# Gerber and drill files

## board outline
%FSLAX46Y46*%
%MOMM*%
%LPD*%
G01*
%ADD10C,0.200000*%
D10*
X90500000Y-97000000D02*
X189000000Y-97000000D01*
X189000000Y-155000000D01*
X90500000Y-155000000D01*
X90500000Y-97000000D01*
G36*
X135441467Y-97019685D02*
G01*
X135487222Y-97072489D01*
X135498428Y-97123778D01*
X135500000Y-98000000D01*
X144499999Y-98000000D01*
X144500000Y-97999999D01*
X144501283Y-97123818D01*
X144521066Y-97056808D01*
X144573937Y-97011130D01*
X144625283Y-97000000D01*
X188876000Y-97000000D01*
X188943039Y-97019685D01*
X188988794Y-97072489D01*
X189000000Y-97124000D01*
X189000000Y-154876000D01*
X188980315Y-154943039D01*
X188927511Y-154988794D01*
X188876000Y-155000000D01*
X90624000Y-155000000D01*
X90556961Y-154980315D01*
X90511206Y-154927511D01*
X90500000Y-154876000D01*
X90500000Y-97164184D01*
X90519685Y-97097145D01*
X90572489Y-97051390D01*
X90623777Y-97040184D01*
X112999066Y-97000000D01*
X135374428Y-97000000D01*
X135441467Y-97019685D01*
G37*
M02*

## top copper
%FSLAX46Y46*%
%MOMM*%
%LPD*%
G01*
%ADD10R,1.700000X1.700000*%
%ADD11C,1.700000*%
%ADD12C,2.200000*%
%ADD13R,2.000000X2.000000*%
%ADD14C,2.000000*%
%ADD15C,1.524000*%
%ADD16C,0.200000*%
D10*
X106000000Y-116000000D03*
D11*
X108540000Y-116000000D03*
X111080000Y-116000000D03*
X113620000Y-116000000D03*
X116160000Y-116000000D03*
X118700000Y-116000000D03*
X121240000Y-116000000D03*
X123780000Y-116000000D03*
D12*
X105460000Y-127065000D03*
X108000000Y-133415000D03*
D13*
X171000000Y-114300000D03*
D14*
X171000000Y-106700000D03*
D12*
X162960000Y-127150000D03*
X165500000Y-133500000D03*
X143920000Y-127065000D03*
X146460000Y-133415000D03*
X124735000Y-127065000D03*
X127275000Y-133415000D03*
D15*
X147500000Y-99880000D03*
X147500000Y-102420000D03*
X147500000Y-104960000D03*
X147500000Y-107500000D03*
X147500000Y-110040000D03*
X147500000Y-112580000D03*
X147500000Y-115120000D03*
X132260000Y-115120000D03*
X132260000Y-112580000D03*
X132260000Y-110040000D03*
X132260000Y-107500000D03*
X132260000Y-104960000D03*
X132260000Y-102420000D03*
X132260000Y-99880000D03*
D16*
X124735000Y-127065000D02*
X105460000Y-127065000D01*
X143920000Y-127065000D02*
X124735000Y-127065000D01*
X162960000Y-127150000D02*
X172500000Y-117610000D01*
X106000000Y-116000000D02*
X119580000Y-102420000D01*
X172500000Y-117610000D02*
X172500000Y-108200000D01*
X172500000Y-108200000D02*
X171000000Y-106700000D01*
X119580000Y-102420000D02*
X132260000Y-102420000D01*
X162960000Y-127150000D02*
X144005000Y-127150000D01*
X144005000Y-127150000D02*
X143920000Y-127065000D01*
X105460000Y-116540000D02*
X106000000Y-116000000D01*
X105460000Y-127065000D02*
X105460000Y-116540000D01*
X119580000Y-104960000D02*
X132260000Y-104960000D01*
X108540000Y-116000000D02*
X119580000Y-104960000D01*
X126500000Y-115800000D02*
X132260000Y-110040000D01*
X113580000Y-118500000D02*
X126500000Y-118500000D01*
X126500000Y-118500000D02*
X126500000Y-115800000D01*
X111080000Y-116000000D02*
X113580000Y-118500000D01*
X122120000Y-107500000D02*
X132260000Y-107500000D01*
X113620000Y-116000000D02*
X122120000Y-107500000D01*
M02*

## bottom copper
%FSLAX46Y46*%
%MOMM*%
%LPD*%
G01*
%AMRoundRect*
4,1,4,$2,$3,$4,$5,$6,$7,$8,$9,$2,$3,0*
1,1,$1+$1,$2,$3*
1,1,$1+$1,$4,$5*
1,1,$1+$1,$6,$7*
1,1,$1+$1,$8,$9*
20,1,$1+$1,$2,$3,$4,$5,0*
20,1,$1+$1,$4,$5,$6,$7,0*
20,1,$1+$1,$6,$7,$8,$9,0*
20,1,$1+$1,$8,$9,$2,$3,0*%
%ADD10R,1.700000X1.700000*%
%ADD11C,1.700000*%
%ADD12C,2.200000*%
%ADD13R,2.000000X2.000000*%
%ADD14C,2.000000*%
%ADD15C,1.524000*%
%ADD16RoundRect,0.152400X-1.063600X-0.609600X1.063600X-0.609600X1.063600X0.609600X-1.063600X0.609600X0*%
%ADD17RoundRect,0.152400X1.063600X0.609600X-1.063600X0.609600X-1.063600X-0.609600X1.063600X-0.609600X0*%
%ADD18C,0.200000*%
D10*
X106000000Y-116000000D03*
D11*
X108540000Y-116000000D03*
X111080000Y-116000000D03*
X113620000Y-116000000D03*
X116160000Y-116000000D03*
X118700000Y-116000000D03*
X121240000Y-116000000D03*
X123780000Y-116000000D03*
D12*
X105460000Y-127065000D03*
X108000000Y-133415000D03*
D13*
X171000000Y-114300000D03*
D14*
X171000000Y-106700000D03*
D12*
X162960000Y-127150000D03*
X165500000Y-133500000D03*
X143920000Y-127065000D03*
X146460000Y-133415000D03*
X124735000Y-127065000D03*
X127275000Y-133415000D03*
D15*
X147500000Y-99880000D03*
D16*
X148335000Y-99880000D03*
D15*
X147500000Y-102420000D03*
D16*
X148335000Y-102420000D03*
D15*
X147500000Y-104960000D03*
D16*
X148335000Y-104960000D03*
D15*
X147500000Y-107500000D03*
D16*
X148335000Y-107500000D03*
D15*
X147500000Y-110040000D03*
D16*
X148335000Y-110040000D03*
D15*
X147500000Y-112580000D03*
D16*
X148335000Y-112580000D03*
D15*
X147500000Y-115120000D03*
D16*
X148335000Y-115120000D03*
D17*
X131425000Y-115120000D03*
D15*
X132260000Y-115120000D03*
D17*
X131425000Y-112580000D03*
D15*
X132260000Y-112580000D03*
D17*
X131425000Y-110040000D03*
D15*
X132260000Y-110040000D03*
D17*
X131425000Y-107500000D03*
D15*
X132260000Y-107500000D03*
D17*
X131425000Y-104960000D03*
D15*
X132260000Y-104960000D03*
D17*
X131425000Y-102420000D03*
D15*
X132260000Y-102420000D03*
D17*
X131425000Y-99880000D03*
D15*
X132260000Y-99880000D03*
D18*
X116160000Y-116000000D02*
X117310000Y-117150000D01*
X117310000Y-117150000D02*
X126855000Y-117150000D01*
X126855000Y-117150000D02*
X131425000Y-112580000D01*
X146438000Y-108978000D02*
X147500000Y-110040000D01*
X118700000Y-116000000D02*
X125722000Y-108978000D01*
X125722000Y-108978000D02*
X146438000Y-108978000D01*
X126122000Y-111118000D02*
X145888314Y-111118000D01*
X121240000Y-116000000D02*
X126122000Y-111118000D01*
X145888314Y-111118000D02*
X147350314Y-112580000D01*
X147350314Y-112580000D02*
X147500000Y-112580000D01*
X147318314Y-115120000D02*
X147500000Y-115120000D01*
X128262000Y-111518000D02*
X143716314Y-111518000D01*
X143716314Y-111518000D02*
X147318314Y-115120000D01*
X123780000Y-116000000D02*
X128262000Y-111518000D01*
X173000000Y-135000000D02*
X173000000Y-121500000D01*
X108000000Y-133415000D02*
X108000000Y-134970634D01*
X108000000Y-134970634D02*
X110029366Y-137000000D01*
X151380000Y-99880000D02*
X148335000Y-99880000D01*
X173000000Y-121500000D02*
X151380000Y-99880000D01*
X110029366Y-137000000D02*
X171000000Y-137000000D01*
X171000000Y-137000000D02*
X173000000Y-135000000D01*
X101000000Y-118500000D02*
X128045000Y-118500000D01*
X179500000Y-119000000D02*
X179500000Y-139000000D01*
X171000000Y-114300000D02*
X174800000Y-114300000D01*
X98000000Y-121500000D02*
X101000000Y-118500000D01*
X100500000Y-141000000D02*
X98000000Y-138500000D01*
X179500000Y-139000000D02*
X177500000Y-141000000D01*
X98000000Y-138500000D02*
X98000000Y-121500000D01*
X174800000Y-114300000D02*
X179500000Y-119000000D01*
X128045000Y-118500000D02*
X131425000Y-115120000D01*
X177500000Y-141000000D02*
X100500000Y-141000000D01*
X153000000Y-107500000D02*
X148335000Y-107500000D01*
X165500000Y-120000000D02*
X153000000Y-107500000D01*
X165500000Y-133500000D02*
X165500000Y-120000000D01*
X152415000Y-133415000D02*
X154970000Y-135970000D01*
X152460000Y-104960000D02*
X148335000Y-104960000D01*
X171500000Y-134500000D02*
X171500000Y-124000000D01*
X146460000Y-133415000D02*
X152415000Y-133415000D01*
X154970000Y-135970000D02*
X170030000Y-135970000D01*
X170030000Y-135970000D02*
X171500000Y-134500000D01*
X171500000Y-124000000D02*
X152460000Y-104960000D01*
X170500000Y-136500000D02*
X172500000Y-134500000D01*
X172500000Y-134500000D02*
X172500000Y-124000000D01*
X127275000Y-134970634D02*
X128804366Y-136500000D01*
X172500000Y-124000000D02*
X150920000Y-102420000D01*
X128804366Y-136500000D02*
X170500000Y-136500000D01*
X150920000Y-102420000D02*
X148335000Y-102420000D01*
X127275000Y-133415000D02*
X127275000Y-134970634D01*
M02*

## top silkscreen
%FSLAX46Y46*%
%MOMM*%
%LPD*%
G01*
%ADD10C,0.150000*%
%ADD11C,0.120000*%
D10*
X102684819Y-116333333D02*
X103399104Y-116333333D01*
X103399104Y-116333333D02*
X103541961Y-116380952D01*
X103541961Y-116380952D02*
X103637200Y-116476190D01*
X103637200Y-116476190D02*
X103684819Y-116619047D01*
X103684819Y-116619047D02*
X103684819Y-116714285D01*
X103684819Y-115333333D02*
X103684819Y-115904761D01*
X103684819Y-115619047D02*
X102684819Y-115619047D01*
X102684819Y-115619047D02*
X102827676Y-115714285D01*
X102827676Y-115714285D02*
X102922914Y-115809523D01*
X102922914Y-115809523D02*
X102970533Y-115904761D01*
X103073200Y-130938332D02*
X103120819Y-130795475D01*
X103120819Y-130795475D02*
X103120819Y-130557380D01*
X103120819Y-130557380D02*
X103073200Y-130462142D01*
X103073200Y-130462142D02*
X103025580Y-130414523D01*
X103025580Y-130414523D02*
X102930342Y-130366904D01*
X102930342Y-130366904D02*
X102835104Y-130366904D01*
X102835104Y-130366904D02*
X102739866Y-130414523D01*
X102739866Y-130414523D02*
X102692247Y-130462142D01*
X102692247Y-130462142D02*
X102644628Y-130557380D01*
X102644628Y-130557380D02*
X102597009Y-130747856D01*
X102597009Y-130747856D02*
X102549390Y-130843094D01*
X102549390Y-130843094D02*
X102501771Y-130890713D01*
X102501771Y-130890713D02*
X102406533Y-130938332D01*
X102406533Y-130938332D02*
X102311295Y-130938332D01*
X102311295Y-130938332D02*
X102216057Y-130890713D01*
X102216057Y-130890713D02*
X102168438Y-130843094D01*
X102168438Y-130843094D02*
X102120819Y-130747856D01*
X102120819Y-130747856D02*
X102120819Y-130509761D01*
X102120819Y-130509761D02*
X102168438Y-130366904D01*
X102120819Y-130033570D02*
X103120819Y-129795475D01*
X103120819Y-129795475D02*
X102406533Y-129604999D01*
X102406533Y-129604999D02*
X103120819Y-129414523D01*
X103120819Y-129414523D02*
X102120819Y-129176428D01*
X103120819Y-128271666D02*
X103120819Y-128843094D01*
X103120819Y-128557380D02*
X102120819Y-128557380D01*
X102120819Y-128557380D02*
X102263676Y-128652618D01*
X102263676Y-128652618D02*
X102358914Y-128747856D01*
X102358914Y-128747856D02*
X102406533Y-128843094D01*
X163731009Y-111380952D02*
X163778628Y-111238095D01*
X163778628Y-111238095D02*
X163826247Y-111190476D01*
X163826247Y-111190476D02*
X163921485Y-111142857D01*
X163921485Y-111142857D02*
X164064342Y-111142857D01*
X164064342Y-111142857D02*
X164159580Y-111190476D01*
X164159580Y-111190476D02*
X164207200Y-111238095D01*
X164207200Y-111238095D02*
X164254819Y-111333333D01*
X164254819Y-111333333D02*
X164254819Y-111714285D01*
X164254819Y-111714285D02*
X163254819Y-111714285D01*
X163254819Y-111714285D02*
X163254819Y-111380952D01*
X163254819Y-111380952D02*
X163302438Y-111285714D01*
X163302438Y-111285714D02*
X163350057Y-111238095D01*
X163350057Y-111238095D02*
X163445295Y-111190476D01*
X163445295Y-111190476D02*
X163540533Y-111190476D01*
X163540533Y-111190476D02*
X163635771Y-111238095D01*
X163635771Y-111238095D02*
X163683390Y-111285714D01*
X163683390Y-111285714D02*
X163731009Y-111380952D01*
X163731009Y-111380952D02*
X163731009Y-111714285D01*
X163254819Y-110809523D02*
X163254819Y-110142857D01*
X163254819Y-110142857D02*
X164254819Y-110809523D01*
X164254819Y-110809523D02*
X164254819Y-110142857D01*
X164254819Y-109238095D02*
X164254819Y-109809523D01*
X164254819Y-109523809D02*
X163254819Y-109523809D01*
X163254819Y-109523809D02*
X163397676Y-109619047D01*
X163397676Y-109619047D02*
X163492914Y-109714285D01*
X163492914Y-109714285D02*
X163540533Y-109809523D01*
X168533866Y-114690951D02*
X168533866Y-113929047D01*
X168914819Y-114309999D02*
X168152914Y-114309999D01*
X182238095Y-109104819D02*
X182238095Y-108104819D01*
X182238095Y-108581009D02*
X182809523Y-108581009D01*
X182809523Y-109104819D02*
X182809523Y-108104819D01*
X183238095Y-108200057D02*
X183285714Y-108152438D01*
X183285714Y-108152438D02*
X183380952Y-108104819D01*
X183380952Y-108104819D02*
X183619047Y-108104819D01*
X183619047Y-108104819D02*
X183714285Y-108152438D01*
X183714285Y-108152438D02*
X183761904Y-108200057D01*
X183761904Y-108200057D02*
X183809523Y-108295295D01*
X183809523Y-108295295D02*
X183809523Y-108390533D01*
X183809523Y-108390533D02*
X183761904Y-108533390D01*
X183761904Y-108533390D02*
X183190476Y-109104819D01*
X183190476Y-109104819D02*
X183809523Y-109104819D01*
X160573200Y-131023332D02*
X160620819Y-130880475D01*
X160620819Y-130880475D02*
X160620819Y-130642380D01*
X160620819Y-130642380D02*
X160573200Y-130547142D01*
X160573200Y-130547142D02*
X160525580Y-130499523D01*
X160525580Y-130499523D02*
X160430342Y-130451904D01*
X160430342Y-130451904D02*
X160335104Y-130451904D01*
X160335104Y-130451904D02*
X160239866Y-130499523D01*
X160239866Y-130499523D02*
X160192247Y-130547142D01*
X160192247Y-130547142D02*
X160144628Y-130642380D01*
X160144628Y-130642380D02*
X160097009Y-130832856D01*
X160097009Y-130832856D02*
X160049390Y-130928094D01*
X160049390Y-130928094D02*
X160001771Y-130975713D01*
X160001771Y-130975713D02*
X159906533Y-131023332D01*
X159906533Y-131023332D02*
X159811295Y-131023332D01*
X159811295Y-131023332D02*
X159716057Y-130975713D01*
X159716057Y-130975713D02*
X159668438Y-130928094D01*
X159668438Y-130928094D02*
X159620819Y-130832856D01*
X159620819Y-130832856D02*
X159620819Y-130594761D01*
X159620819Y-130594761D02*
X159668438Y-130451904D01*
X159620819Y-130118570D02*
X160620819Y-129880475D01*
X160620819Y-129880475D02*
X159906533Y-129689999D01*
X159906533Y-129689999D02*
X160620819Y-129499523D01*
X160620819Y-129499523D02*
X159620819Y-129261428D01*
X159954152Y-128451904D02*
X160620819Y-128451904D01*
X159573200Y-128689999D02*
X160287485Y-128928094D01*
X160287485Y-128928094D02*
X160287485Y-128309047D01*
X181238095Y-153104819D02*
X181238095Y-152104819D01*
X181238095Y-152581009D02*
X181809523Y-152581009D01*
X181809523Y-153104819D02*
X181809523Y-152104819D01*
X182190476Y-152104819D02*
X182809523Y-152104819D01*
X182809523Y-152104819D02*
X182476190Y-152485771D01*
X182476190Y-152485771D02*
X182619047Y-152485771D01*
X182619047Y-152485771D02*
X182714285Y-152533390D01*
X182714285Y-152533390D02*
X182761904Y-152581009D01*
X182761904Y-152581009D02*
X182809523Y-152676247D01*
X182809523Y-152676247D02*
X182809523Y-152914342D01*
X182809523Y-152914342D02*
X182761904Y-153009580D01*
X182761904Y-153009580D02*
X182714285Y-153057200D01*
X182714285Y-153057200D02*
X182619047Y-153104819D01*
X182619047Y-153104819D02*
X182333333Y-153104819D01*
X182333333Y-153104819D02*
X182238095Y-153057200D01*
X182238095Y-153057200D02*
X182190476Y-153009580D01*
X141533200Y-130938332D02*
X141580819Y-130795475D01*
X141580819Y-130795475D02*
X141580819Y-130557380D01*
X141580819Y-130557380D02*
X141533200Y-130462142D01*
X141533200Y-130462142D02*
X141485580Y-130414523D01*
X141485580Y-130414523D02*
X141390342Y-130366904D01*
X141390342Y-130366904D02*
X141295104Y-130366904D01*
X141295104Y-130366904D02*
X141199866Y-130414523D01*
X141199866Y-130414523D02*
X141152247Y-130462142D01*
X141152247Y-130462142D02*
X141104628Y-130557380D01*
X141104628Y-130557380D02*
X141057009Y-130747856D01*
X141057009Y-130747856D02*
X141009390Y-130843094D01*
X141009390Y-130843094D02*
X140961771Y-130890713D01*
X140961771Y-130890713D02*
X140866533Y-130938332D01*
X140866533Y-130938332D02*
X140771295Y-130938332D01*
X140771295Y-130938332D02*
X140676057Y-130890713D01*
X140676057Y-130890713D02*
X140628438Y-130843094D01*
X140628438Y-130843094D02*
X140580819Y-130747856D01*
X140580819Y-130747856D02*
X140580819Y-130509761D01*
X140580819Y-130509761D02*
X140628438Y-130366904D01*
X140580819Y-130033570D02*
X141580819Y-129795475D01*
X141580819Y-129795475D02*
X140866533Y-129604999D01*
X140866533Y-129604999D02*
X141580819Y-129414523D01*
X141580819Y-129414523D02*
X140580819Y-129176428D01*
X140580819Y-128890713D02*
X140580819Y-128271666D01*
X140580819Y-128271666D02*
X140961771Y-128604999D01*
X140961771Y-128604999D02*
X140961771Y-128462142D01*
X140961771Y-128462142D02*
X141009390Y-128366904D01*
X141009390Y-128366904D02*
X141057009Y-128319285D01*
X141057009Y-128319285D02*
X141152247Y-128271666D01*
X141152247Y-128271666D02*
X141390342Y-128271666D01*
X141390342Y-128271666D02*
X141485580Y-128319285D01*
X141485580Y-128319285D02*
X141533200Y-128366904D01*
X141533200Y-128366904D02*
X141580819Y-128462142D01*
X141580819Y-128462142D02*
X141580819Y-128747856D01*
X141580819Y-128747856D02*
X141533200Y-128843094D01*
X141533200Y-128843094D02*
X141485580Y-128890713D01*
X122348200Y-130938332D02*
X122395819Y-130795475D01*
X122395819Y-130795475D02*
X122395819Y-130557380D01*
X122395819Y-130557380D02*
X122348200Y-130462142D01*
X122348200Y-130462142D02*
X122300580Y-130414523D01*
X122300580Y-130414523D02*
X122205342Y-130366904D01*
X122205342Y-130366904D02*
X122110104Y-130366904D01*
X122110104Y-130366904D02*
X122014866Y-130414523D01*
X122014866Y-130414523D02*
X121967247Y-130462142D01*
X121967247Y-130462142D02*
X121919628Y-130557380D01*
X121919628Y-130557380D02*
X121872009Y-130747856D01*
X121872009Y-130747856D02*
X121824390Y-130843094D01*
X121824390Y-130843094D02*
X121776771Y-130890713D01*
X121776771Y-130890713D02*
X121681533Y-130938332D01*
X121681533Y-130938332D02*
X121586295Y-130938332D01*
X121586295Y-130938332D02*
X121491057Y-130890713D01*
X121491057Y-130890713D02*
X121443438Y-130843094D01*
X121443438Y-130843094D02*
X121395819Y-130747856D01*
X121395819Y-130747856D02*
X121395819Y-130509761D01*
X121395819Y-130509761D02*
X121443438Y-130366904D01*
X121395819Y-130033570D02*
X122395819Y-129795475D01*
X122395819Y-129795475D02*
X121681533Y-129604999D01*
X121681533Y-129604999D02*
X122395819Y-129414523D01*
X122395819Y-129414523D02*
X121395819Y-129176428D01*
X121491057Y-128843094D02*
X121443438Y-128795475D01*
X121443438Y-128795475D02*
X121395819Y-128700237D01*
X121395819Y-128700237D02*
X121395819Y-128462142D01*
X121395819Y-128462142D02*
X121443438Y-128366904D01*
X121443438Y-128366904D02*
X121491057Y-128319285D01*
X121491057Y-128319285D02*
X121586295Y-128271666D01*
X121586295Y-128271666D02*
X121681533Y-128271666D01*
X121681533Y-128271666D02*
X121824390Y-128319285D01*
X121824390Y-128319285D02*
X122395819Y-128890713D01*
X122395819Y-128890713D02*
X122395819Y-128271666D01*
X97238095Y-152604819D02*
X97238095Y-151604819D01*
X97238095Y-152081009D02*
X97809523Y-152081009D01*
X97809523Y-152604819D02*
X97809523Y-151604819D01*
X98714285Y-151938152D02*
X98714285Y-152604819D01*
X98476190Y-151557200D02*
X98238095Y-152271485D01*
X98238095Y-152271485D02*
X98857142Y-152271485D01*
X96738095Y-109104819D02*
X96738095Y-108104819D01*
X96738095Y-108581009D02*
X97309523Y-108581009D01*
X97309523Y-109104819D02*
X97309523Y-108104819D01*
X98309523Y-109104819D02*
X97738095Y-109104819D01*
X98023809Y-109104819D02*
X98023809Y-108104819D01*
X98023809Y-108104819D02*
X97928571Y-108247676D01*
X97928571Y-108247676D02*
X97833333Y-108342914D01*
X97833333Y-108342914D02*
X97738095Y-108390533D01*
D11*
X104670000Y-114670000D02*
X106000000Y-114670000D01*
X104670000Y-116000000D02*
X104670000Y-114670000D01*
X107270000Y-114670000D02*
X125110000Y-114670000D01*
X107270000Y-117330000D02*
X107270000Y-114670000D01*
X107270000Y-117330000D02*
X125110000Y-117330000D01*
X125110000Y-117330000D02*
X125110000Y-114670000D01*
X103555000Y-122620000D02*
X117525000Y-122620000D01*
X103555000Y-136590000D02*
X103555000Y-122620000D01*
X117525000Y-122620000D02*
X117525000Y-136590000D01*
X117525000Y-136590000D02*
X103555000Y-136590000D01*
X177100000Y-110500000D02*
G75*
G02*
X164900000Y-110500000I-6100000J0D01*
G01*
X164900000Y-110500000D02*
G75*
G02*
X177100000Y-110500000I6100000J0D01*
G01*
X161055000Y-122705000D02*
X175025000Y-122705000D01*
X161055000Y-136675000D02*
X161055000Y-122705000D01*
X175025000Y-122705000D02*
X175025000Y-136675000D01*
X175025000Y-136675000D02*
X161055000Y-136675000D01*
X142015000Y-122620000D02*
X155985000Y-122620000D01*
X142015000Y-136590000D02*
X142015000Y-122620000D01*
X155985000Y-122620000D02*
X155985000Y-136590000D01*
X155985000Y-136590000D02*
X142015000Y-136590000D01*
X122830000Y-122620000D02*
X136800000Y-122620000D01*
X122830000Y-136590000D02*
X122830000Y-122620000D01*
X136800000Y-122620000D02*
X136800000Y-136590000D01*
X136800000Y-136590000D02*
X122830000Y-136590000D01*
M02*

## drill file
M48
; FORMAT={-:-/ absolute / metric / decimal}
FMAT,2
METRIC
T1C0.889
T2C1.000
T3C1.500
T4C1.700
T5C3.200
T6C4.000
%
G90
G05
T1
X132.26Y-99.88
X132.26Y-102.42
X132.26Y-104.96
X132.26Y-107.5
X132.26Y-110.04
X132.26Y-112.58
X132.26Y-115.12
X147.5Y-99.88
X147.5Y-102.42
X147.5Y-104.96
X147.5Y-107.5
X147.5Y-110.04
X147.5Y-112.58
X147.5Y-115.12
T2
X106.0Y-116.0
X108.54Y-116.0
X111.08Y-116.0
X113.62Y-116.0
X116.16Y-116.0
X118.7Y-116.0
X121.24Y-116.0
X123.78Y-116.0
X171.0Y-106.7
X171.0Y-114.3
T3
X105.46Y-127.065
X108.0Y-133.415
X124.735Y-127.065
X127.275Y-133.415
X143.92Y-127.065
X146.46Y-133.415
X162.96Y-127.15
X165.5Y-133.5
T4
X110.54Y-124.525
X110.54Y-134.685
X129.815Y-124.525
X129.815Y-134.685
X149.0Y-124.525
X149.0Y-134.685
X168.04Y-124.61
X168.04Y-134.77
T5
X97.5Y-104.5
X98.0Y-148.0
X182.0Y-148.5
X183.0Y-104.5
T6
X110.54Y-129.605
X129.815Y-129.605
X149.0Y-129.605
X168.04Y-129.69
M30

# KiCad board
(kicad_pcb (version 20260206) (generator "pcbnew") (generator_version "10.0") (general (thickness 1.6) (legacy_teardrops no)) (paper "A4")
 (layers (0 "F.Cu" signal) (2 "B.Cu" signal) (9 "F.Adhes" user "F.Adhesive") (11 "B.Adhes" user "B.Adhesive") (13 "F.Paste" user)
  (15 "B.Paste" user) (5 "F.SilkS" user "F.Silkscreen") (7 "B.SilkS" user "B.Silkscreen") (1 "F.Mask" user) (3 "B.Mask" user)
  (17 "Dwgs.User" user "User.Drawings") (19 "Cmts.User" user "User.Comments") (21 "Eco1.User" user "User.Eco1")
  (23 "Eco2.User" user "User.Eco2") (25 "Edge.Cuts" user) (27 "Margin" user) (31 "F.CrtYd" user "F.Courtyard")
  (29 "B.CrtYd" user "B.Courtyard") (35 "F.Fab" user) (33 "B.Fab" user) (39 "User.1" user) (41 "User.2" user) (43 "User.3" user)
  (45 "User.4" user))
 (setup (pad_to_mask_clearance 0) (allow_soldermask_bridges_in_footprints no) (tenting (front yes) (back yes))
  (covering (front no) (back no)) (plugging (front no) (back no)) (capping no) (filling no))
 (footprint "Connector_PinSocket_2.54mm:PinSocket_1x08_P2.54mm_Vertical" (layer "F.Cu") (at 106 116 90)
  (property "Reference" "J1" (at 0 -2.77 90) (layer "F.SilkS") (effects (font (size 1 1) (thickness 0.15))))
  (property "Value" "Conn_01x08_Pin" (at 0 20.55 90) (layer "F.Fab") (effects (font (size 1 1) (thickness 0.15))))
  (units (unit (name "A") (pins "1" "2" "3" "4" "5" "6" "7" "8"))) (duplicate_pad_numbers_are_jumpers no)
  (fp_line (start 1.33 -1.33) (end 1.33 0) (stroke (width 0.12) (type solid)) (layer "F.SilkS"))
  (fp_line (start 0 -1.33) (end 1.33 -1.33) (stroke (width 0.12) (type solid)) (layer "F.SilkS"))
  (fp_line (start 1.33 1.27) (end 1.33 19.11) (stroke (width 0.12) (type solid)) (layer "F.SilkS"))
  (fp_line (start -1.33 1.27) (end 1.33 1.27) (stroke (width 0.12) (type solid)) (layer "F.SilkS"))
  (fp_line (start -1.33 1.27) (end -1.33 19.11) (stroke (width 0.12) (type solid)) (layer "F.SilkS"))
  (fp_line (start -1.33 19.11) (end 1.33 19.11) (stroke (width 0.12) (type solid)) (layer "F.SilkS"))
  (pad "1" thru_hole rect (at 0 0 90) (size 1.7 1.7) (drill 1) (layers "*.Cu" "*.Mask") (remove_unused_layers no) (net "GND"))
  (pad "2" thru_hole circle (at 0 2.54 90) (size 1.7 1.7) (drill 1) (layers "*.Cu" "*.Mask") (remove_unused_layers no) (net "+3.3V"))
  (pad "3" thru_hole circle (at 0 5.08 90) (size 1.7 1.7) (drill 1) (layers "*.Cu" "*.Mask") (remove_unused_layers no) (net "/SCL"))
  (pad "4" thru_hole circle (at 0 7.62 90) (size 1.7 1.7) (drill 1) (layers "*.Cu" "*.Mask") (remove_unused_layers no) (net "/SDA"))
  (pad "5" thru_hole circle (at 0 10.16 90) (size 1.7 1.7) (drill 1) (layers "*.Cu" "*.Mask") (remove_unused_layers no) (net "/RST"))
  (pad "6" thru_hole circle (at 0 12.7 90) (size 1.7 1.7) (drill 1) (layers "*.Cu" "*.Mask") (remove_unused_layers no) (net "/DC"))
  (pad "7" thru_hole circle (at 0 15.24 90) (size 1.7 1.7) (drill 1) (layers "*.Cu" "*.Mask") (remove_unused_layers no) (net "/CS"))
  (pad "8" thru_hole circle (at 0 17.78 90) (size 1.7 1.7) (drill 1) (layers "*.Cu" "*.Mask") (remove_unused_layers no) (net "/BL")))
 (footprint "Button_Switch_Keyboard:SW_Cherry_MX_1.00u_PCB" (layer "F.Cu") (at 105.46 127.065 90)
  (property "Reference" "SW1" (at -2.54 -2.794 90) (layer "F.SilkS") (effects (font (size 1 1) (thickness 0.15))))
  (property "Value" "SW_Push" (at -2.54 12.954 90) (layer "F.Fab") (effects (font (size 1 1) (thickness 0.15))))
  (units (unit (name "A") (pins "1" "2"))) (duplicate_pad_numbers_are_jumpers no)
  (fp_line (start 4.445 -1.905) (end 4.445 12.065) (stroke (width 0.12) (type solid)) (layer "F.SilkS"))
  (fp_line (start -9.525 -1.905) (end 4.445 -1.905) (stroke (width 0.12) (type solid)) (layer "F.SilkS"))
  (fp_line (start 4.445 12.065) (end -9.525 12.065) (stroke (width 0.12) (type solid)) (layer "F.SilkS"))
  (fp_line (start -9.525 12.065) (end -9.525 -1.905) (stroke (width 0.12) (type solid)) (layer "F.SilkS"))
  (pad "" np_thru_hole circle (at -7.62 5.08 90) (size 1.7 1.7) (drill 1.7) (layers "*.Cu" "*.Mask"))
  (pad "" np_thru_hole circle (at -2.54 5.08 90) (size 4 4) (drill 4) (layers "*.Cu" "*.Mask"))
  (pad "" np_thru_hole circle (at 2.54 5.08 90) (size 1.7 1.7) (drill 1.7) (layers "*.Cu" "*.Mask"))
  (pad "1" thru_hole circle (at 0 0 90) (size 2.2 2.2) (drill 1.5) (layers "*.Cu" "*.Mask") (remove_unused_layers no) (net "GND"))
  (pad "2" thru_hole circle (at -6.35 2.54 90) (size 2.2 2.2) (drill 1.5) (layers "*.Cu" "*.Mask") (remove_unused_layers no)
   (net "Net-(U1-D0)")))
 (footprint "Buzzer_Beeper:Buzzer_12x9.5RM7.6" (layer "F.Cu") (at 171 114.3 90)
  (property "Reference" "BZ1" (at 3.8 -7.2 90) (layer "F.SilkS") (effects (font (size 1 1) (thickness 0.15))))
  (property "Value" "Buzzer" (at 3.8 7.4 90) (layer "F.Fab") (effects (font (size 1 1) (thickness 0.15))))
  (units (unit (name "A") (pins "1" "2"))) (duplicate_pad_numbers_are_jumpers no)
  (fp_circle (center 3.8 0) (end 9.9 0) (stroke (width 0.12) (type solid)) (fill no) (layer "F.SilkS"))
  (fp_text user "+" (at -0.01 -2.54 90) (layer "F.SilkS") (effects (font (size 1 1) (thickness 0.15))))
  (pad "1" thru_hole rect (at 0 0 90) (size 2 2) (drill 1) (layers "*.Cu" "*.Mask") (remove_unused_layers no) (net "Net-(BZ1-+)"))
  (pad "2" thru_hole circle (at 7.6 0 90) (size 2 2) (drill 1) (layers "*.Cu" "*.Mask") (remove_unused_layers no) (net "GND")))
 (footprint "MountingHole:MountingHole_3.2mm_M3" (layer "F.Cu") (at 183 104.5 180)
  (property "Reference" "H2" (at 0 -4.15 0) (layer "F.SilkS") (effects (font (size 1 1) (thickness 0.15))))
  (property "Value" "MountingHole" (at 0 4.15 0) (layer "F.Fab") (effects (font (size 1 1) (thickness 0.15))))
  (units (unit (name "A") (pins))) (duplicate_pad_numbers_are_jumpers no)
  (pad "" np_thru_hole circle (at 0 0 180) (size 3.2 3.2) (drill 3.2) (layers "*.Cu" "*.Mask")))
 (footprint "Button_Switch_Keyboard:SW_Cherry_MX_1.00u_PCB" (layer "F.Cu") (at 162.96 127.15 90)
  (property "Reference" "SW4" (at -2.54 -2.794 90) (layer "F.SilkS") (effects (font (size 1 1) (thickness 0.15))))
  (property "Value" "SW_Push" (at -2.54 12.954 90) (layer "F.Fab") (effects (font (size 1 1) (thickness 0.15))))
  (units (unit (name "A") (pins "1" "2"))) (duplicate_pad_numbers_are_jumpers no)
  (fp_line (start 4.445 -1.905) (end 4.445 12.065) (stroke (width 0.12) (type solid)) (layer "F.SilkS"))
  (fp_line (start -9.525 -1.905) (end 4.445 -1.905) (stroke (width 0.12) (type solid)) (layer "F.SilkS"))
  (fp_line (start 4.445 12.065) (end -9.525 12.065) (stroke (width 0.12) (type solid)) (layer "F.SilkS"))
  (fp_line (start -9.525 12.065) (end -9.525 -1.905) (stroke (width 0.12) (type solid)) (layer "F.SilkS"))
  (pad "" np_thru_hole circle (at -7.62 5.08 90) (size 1.7 1.7) (drill 1.7) (layers "*.Cu" "*.Mask"))
  (pad "" np_thru_hole circle (at -2.54 5.08 90) (size 4 4) (drill 4) (layers "*.Cu" "*.Mask"))
  (pad "" np_thru_hole circle (at 2.54 5.08 90) (size 1.7 1.7) (drill 1.7) (layers "*.Cu" "*.Mask"))
  (pad "1" thru_hole circle (at 0 0 90) (size 2.2 2.2) (drill 1.5) (layers "*.Cu" "*.Mask") (remove_unused_layers no) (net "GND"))
  (pad "2" thru_hole circle (at -6.35 2.54 90) (size 2.2 2.2) (drill 1.5) (layers "*.Cu" "*.Mask") (remove_unused_layers no)
   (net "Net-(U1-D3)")))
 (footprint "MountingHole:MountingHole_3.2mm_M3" (layer "F.Cu") (at 182 148.5 180)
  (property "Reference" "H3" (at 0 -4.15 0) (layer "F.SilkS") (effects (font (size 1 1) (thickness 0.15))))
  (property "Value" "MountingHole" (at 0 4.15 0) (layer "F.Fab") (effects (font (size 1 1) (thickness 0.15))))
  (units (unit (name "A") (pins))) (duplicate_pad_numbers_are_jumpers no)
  (pad "" np_thru_hole circle (at 0 0 180) (size 3.2 3.2) (drill 3.2) (layers "*.Cu" "*.Mask")))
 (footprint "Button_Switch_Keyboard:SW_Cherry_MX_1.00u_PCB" (layer "F.Cu") (at 143.92 127.065 90)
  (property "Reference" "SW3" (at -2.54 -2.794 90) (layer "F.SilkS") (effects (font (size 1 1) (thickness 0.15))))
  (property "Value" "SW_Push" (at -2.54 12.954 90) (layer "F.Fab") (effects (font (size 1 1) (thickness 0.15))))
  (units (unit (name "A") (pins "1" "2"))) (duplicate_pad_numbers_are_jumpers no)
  (fp_line (start 4.445 -1.905) (end 4.445 12.065) (stroke (width 0.12) (type solid)) (layer "F.SilkS"))
  (fp_line (start -9.525 -1.905) (end 4.445 -1.905) (stroke (width 0.12) (type solid)) (layer "F.SilkS"))
  (fp_line (start 4.445 12.065) (end -9.525 12.065) (stroke (width 0.12) (type solid)) (layer "F.SilkS"))
  (fp_line (start -9.525 12.065) (end -9.525 -1.905) (stroke (width 0.12) (type solid)) (layer "F.SilkS"))
  (pad "" np_thru_hole circle (at -7.62 5.08 90) (size 1.7 1.7) (drill 1.7) (layers "*.Cu" "*.Mask"))
  (pad "" np_thru_hole circle (at -2.54 5.08 90) (size 4 4) (drill 4) (layers "*.Cu" "*.Mask"))
  (pad "" np_thru_hole circle (at 2.54 5.08 90) (size 1.7 1.7) (drill 1.7) (layers "*.Cu" "*.Mask"))
  (pad "1" thru_hole circle (at 0 0 90) (size 2.2 2.2) (drill 1.5) (layers "*.Cu" "*.Mask") (remove_unused_layers no) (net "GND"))
  (pad "2" thru_hole circle (at -6.35 2.54 90) (size 2.2 2.2) (drill 1.5) (layers "*.Cu" "*.Mask") (remove_unused_layers no)
   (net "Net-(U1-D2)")))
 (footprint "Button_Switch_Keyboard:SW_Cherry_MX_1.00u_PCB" (layer "F.Cu") (at 124.735 127.065 90)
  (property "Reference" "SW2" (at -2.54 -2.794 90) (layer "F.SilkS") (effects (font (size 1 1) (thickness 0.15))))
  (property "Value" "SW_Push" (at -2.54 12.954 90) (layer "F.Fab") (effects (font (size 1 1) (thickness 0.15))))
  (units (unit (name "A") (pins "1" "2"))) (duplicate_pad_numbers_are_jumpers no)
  (fp_line (start 4.445 -1.905) (end 4.445 12.065) (stroke (width 0.12) (type solid)) (layer "F.SilkS"))
  (fp_line (start -9.525 -1.905) (end 4.445 -1.905) (stroke (width 0.12) (type solid)) (layer "F.SilkS"))
  (fp_line (start 4.445 12.065) (end -9.525 12.065) (stroke (width 0.12) (type solid)) (layer "F.SilkS"))
  (fp_line (start -9.525 12.065) (end -9.525 -1.905) (stroke (width 0.12) (type solid)) (layer "F.SilkS"))
  (pad "" np_thru_hole circle (at -7.62 5.08 90) (size 1.7 1.7) (drill 1.7) (layers "*.Cu" "*.Mask"))
  (pad "" np_thru_hole circle (at -2.54 5.08 90) (size 4 4) (drill 4) (layers "*.Cu" "*.Mask"))
  (pad "" np_thru_hole circle (at 2.54 5.08 90) (size 1.7 1.7) (drill 1.7) (layers "*.Cu" "*.Mask"))
  (pad "1" thru_hole circle (at 0 0 90) (size 2.2 2.2) (drill 1.5) (layers "*.Cu" "*.Mask") (remove_unused_layers no) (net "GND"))
  (pad "2" thru_hole circle (at -6.35 2.54 90) (size 2.2 2.2) (drill 1.5) (layers "*.Cu" "*.Mask") (remove_unused_layers no)
   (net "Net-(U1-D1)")))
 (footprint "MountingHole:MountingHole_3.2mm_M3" (layer "F.Cu") (at 98 148 180)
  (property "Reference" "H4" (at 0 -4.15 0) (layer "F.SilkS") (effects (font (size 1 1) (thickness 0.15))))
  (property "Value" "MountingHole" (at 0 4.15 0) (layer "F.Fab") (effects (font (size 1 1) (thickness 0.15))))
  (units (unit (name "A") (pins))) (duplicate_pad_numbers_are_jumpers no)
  (pad "" np_thru_hole circle (at 0 0 180) (size 3.2 3.2) (drill 3.2) (layers "*.Cu" "*.Mask")))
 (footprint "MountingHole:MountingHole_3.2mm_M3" (layer "F.Cu") (at 97.5 104.5 180)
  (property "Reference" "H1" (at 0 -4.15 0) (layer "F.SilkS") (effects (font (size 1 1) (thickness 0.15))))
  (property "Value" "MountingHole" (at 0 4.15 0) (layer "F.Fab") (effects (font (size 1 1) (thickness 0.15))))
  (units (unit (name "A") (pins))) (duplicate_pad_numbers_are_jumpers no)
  (pad "" np_thru_hole circle (at 0 0 180) (size 3.2 3.2) (drill 3.2) (layers "*.Cu" "*.Mask")))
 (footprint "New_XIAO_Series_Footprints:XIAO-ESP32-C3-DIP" (layer "B.Cu") (at 139.88 107.5 90)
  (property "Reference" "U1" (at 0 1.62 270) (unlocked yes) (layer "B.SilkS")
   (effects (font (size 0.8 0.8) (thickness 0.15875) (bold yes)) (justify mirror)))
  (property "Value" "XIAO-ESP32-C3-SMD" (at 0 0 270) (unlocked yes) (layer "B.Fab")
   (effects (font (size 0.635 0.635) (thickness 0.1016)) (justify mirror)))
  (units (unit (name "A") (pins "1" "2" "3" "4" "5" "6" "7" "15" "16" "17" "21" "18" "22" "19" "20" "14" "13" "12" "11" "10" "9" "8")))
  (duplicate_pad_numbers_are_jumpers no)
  (pad "1" thru_hole circle (at 7.62 7.62) (size 1.524 1.524) (drill 0.889) (layers "*.Cu" "*.Mask") (remove_unused_layers no)
   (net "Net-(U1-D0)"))
  (pad "1" smd roundrect (at 7.62 8.455) (size 2.432 1.524) (layers "B.Cu" "B.Mask") (roundrect_rratio 0.1) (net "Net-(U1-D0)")
   (thermal_bridge_angle 45))
  (pad "2" thru_hole circle (at 5.08 7.62) (size 1.524 1.524) (drill 0.889) (layers "*.Cu" "*.Mask") (remove_unused_layers no)
   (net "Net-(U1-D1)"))
  (pad "2" smd roundrect (at 5.08 8.455) (size 2.432 1.524) (layers "B.Cu" "B.Mask") (roundrect_rratio 0.1) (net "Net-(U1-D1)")
   (thermal_bridge_angle 45))
  (pad "3" thru_hole circle (at 2.54 7.62) (size 1.524 1.524) (drill 0.889) (layers "*.Cu" "*.Mask") (remove_unused_layers no)
   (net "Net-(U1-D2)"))
  (pad "3" smd roundrect (at 2.54 8.455) (size 2.432 1.524) (layers "B.Cu" "B.Mask") (roundrect_rratio 0.1) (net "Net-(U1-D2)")
   (thermal_bridge_angle 45))
  (pad "4" thru_hole circle (at 0 7.62) (size 1.524 1.524) (drill 0.889) (layers "*.Cu" "*.Mask") (remove_unused_layers no)
   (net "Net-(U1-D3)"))
  (pad "4" smd roundrect (at 0 8.455) (size 2.432 1.524) (layers "B.Cu" "B.Mask") (roundrect_rratio 0.1) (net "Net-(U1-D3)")
   (thermal_bridge_angle 45))
  (pad "5" thru_hole circle (at -2.54 7.62) (size 1.524 1.524) (drill 0.889) (layers "*.Cu" "*.Mask") (remove_unused_layers no) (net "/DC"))
  (pad "5" smd roundrect (at -2.54 8.455) (size 2.432 1.524) (layers "B.Cu" "B.Mask") (roundrect_rratio 0.1) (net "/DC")
   (thermal_bridge_angle 45))
  (pad "6" thru_hole circle (at -5.08 7.62) (size 1.524 1.524) (drill 0.889) (layers "*.Cu" "*.Mask") (remove_unused_layers no) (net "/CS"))
  (pad "6" smd roundrect (at -5.08 8.455) (size 2.432 1.524) (layers "B.Cu" "B.Mask") (roundrect_rratio 0.1) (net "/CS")
   (thermal_bridge_angle 45))
  (pad "7" thru_hole circle (at -7.62 7.62) (size 1.524 1.524) (drill 0.889) (layers "*.Cu" "*.Mask") (remove_unused_layers no) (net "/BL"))
  (pad "7" smd roundrect (at -7.62 8.455) (size 2.432 1.524) (layers "B.Cu" "B.Mask") (roundrect_rratio 0.1) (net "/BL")
   (thermal_bridge_angle 45))
  (pad "8" smd roundrect (at -7.62 -8.455 180) (size 2.432 1.524) (layers "B.Cu" "B.Mask") (roundrect_rratio 0.1) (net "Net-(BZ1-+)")
   (thermal_bridge_angle 45))
  (pad "8" thru_hole circle (at -7.62 -7.62 180) (size 1.524 1.524) (drill 0.889) (layers "*.Cu" "*.Mask") (remove_unused_layers no)
   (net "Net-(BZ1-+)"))
  (pad "9" smd roundrect (at -5.08 -8.455 180) (size 2.432 1.524) (layers "B.Cu" "B.Mask") (roundrect_rratio 0.1) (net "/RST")
   (thermal_bridge_angle 45))
  (pad "9" thru_hole circle (at -5.08 -7.62 180) (size 1.524 1.524) (drill 0.889) (layers "*.Cu" "*.Mask") (remove_unused_layers no)
   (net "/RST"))
  (pad "10" smd roundrect (at -2.54 -8.455 180) (size 2.432 1.524) (layers "B.Cu" "B.Mask") (roundrect_rratio 0.1) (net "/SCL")
   (thermal_bridge_angle 45))
  (pad "10" thru_hole circle (at -2.54 -7.62 180) (size 1.524 1.524) (drill 0.889) (layers "*.Cu" "*.Mask") (remove_unused_layers no)
   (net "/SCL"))
  (pad "11" smd roundrect (at 0 -8.455 180) (size 2.432 1.524) (layers "B.Cu" "B.Mask") (roundrect_rratio 0.1) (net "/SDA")
   (thermal_bridge_angle 45))
  (pad "11" thru_hole circle (at 0 -7.62 180) (size 1.524 1.524) (drill 0.889) (layers "*.Cu" "*.Mask") (remove_unused_layers no)
   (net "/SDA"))
  (pad "12" smd roundrect (at 2.54 -8.455 180) (size 2.432 1.524) (layers "B.Cu" "B.Mask") (roundrect_rratio 0.1) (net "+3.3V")
   (thermal_bridge_angle 45))
  (pad "12" thru_hole circle (at 2.54 -7.62 180) (size 1.524 1.524) (drill 0.889) (layers "*.Cu" "*.Mask") (remove_unused_layers no)
   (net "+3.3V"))
  (pad "13" smd roundrect (at 5.08 -8.455 180) (size 2.432 1.524) (layers "B.Cu" "B.Mask") (roundrect_rratio 0.1) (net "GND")
   (thermal_bridge_angle 45))
  (pad "13" thru_hole circle (at 5.08 -7.62 180) (size 1.524 1.524) (drill 0.889) (layers "*.Cu" "*.Mask") (remove_unused_layers no)
   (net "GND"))
  (pad "14" smd roundrect (at 7.62 -8.455 180) (size 2.432 1.524) (layers "B.Cu" "B.Mask") (roundrect_rratio 0.1)
   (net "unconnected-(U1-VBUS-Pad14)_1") (thermal_bridge_angle 45))
  (pad "14" thru_hole circle (at 7.62 -7.62 180) (size 1.524 1.524) (drill 0.889) (layers "*.Cu" "*.Mask") (remove_unused_layers no)
   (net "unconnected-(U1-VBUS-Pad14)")))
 (gr_rect (start 90.5 97) (end 189 155) (stroke (width 0.2) (type default)) (fill no) (layer "Edge.Cuts"))
 (segment (start 124.735 127.065) (end 105.46 127.065) (width 0.2) (layer "F.Cu") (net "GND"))
 (segment (start 143.92 127.065) (end 124.735 127.065) (width 0.2) (layer "F.Cu") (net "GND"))
 (segment (start 162.96 127.15) (end 172.5 117.61) (width 0.2) (layer "F.Cu") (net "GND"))
 (segment (start 106 116) (end 119.58 102.42) (width 0.2) (layer "F.Cu") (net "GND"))
 (segment (start 172.5 117.61) (end 172.5 108.2) (width 0.2) (layer "F.Cu") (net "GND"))
 (segment (start 172.5 108.2) (end 171 106.7) (width 0.2) (layer "F.Cu") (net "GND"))
 (segment (start 119.58 102.42) (end 132.26 102.42) (width 0.2) (layer "F.Cu") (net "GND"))
 (segment (start 162.96 127.15) (end 144.005 127.15) (width 0.2) (layer "F.Cu") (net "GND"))
 (segment (start 144.005 127.15) (end 143.92 127.065) (width 0.2) (layer "F.Cu") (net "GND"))
 (segment (start 105.46 116.54) (end 106 116) (width 0.2) (layer "F.Cu") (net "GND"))
 (segment (start 105.46 127.065) (end 105.46 116.54) (width 0.2) (layer "F.Cu") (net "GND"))
 (segment (start 119.58 104.96) (end 132.26 104.96) (width 0.2) (layer "F.Cu") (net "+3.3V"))
 (segment (start 108.54 116) (end 119.58 104.96) (width 0.2) (layer "F.Cu") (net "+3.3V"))
 (segment (start 126.5 115.8) (end 132.26 110.04) (width 0.2) (layer "F.Cu") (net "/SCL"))
 (segment (start 113.58 118.5) (end 126.5 118.5) (width 0.2) (layer "F.Cu") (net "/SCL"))
 (segment (start 126.5 118.5) (end 126.5 115.8) (width 0.2) (layer "F.Cu") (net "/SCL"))
 (segment (start 111.08 116) (end 113.58 118.5) (width 0.2) (layer "F.Cu") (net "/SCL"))
 (segment (start 122.12 107.5) (end 132.26 107.5) (width 0.2) (layer "F.Cu") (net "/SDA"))
 (segment (start 113.62 116) (end 122.12 107.5) (width 0.2) (layer "F.Cu") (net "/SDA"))
 (segment (start 116.16 116) (end 117.31 117.15) (width 0.2) (layer "B.Cu") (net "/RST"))
 (segment (start 117.31 117.15) (end 126.855 117.15) (width 0.2) (layer "B.Cu") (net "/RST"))
 (segment (start 126.855 117.15) (end 131.425 112.58) (width 0.2) (layer "B.Cu") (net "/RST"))
 (segment (start 146.438 108.978) (end 147.5 110.04) (width 0.2) (layer "B.Cu") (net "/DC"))
 (segment (start 118.7 116) (end 125.722 108.978) (width 0.2) (layer "B.Cu") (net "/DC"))
 (segment (start 125.722 108.978) (end 146.438 108.978) (width 0.2) (layer "B.Cu") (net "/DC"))
 (segment (start 126.122 111.118) (end 145.888314 111.118) (width 0.2) (layer "B.Cu") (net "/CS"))
 (segment (start 121.24 116) (end 126.122 111.118) (width 0.2) (layer "B.Cu") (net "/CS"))
 (segment (start 145.888314 111.118) (end 147.350314 112.58) (width 0.2) (layer "B.Cu") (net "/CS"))
 (segment (start 147.350314 112.58) (end 147.5 112.58) (width 0.2) (layer "B.Cu") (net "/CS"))
 (segment (start 147.318314 115.12) (end 147.5 115.12) (width 0.2) (layer "B.Cu") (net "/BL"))
 (segment (start 128.262 111.518) (end 143.716314 111.518) (width 0.2) (layer "B.Cu") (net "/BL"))
 (segment (start 143.716314 111.518) (end 147.318314 115.12) (width 0.2) (layer "B.Cu") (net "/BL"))
 (segment (start 123.78 116) (end 128.262 111.518) (width 0.2) (layer "B.Cu") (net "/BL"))
 (segment (start 173 135) (end 173 121.5) (width 0.2) (layer "B.Cu") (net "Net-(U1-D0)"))
 (segment (start 108 133.415) (end 108 134.970634) (width 0.2) (layer "B.Cu") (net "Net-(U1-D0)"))
 (segment (start 108 134.970634) (end 110.029366 137) (width 0.2) (layer "B.Cu") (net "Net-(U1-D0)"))
 (segment (start 151.38 99.88) (end 148.335 99.88) (width 0.2) (layer "B.Cu") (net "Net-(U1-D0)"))
 (segment (start 173 121.5) (end 151.38 99.88) (width 0.2) (layer "B.Cu") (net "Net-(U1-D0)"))
 (segment (start 110.029366 137) (end 171 137) (width 0.2) (layer "B.Cu") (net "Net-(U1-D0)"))
 (segment (start 171 137) (end 173 135) (width 0.2) (layer "B.Cu") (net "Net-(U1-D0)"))
 (segment (start 101 118.5) (end 128.045 118.5) (width 0.2) (layer "B.Cu") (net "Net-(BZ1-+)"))
 (segment (start 179.5 119) (end 179.5 139) (width 0.2) (layer "B.Cu") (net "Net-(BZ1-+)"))
 (segment (start 171 114.3) (end 174.8 114.3) (width 0.2) (layer "B.Cu") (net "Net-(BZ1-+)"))
 (segment (start 98 121.5) (end 101 118.5) (width 0.2) (layer "B.Cu") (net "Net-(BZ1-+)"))
 (segment (start 100.5 141) (end 98 138.5) (width 0.2) (layer "B.Cu") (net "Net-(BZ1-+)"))
 (segment (start 179.5 139) (end 177.5 141) (width 0.2) (layer "B.Cu") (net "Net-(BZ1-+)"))
 (segment (start 98 138.5) (end 98 121.5) (width 0.2) (layer "B.Cu") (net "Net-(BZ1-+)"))
 (segment (start 174.8 114.3) (end 179.5 119) (width 0.2) (layer "B.Cu") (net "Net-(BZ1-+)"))
 (segment (start 128.045 118.5) (end 131.425 115.12) (width 0.2) (layer "B.Cu") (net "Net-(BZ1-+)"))
 (segment (start 177.5 141) (end 100.5 141) (width 0.2) (layer "B.Cu") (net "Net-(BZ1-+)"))
 (segment (start 153 107.5) (end 148.335 107.5) (width 0.2) (layer "B.Cu") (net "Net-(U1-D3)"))
 (segment (start 165.5 120) (end 153 107.5) (width 0.2) (layer "B.Cu") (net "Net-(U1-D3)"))
 (segment (start 165.5 133.5) (end 165.5 120) (width 0.2) (layer "B.Cu") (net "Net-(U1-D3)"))
 (segment (start 152.415 133.415) (end 154.97 135.97) (width 0.2) (layer "B.Cu") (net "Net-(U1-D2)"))
 (segment (start 152.46 104.96) (end 148.335 104.96) (width 0.2) (layer "B.Cu") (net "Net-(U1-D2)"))
 (segment (start 171.5 134.5) (end 171.5 124) (width 0.2) (layer "B.Cu") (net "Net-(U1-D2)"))
 (segment (start 146.46 133.415) (end 152.415 133.415) (width 0.2) (layer "B.Cu") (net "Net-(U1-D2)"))
 (segment (start 154.97 135.97) (end 170.03 135.97) (width 0.2) (layer "B.Cu") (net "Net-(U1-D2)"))
 (segment (start 170.03 135.97) (end 171.5 134.5) (width 0.2) (layer "B.Cu") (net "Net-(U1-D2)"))
 (segment (start 171.5 124) (end 152.46 104.96) (width 0.2) (layer "B.Cu") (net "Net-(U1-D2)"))
 (segment (start 170.5 136.5) (end 172.5 134.5) (width 0.2) (layer "B.Cu") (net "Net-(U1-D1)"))
 (segment (start 172.5 134.5) (end 172.5 124) (width 0.2) (layer "B.Cu") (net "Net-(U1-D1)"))
 (segment (start 127.275 134.970634) (end 128.804366 136.5) (width 0.2) (layer "B.Cu") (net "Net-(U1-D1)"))
 (segment (start 172.5 124) (end 150.92 102.42) (width 0.2) (layer "B.Cu") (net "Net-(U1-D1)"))
 (segment (start 128.804366 136.5) (end 170.5 136.5) (width 0.2) (layer "B.Cu") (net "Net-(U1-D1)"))
 (segment (start 150.92 102.42) (end 148.335 102.42) (width 0.2) (layer "B.Cu") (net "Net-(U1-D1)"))
 (segment (start 127.275 133.415) (end 127.275 134.970634) (width 0.2) (layer "B.Cu") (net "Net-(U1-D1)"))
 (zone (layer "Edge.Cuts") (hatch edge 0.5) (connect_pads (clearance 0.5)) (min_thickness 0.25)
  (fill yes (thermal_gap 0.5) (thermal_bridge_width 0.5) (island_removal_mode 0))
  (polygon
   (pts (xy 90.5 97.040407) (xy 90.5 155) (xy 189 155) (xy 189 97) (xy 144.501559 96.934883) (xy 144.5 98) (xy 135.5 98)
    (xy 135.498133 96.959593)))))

